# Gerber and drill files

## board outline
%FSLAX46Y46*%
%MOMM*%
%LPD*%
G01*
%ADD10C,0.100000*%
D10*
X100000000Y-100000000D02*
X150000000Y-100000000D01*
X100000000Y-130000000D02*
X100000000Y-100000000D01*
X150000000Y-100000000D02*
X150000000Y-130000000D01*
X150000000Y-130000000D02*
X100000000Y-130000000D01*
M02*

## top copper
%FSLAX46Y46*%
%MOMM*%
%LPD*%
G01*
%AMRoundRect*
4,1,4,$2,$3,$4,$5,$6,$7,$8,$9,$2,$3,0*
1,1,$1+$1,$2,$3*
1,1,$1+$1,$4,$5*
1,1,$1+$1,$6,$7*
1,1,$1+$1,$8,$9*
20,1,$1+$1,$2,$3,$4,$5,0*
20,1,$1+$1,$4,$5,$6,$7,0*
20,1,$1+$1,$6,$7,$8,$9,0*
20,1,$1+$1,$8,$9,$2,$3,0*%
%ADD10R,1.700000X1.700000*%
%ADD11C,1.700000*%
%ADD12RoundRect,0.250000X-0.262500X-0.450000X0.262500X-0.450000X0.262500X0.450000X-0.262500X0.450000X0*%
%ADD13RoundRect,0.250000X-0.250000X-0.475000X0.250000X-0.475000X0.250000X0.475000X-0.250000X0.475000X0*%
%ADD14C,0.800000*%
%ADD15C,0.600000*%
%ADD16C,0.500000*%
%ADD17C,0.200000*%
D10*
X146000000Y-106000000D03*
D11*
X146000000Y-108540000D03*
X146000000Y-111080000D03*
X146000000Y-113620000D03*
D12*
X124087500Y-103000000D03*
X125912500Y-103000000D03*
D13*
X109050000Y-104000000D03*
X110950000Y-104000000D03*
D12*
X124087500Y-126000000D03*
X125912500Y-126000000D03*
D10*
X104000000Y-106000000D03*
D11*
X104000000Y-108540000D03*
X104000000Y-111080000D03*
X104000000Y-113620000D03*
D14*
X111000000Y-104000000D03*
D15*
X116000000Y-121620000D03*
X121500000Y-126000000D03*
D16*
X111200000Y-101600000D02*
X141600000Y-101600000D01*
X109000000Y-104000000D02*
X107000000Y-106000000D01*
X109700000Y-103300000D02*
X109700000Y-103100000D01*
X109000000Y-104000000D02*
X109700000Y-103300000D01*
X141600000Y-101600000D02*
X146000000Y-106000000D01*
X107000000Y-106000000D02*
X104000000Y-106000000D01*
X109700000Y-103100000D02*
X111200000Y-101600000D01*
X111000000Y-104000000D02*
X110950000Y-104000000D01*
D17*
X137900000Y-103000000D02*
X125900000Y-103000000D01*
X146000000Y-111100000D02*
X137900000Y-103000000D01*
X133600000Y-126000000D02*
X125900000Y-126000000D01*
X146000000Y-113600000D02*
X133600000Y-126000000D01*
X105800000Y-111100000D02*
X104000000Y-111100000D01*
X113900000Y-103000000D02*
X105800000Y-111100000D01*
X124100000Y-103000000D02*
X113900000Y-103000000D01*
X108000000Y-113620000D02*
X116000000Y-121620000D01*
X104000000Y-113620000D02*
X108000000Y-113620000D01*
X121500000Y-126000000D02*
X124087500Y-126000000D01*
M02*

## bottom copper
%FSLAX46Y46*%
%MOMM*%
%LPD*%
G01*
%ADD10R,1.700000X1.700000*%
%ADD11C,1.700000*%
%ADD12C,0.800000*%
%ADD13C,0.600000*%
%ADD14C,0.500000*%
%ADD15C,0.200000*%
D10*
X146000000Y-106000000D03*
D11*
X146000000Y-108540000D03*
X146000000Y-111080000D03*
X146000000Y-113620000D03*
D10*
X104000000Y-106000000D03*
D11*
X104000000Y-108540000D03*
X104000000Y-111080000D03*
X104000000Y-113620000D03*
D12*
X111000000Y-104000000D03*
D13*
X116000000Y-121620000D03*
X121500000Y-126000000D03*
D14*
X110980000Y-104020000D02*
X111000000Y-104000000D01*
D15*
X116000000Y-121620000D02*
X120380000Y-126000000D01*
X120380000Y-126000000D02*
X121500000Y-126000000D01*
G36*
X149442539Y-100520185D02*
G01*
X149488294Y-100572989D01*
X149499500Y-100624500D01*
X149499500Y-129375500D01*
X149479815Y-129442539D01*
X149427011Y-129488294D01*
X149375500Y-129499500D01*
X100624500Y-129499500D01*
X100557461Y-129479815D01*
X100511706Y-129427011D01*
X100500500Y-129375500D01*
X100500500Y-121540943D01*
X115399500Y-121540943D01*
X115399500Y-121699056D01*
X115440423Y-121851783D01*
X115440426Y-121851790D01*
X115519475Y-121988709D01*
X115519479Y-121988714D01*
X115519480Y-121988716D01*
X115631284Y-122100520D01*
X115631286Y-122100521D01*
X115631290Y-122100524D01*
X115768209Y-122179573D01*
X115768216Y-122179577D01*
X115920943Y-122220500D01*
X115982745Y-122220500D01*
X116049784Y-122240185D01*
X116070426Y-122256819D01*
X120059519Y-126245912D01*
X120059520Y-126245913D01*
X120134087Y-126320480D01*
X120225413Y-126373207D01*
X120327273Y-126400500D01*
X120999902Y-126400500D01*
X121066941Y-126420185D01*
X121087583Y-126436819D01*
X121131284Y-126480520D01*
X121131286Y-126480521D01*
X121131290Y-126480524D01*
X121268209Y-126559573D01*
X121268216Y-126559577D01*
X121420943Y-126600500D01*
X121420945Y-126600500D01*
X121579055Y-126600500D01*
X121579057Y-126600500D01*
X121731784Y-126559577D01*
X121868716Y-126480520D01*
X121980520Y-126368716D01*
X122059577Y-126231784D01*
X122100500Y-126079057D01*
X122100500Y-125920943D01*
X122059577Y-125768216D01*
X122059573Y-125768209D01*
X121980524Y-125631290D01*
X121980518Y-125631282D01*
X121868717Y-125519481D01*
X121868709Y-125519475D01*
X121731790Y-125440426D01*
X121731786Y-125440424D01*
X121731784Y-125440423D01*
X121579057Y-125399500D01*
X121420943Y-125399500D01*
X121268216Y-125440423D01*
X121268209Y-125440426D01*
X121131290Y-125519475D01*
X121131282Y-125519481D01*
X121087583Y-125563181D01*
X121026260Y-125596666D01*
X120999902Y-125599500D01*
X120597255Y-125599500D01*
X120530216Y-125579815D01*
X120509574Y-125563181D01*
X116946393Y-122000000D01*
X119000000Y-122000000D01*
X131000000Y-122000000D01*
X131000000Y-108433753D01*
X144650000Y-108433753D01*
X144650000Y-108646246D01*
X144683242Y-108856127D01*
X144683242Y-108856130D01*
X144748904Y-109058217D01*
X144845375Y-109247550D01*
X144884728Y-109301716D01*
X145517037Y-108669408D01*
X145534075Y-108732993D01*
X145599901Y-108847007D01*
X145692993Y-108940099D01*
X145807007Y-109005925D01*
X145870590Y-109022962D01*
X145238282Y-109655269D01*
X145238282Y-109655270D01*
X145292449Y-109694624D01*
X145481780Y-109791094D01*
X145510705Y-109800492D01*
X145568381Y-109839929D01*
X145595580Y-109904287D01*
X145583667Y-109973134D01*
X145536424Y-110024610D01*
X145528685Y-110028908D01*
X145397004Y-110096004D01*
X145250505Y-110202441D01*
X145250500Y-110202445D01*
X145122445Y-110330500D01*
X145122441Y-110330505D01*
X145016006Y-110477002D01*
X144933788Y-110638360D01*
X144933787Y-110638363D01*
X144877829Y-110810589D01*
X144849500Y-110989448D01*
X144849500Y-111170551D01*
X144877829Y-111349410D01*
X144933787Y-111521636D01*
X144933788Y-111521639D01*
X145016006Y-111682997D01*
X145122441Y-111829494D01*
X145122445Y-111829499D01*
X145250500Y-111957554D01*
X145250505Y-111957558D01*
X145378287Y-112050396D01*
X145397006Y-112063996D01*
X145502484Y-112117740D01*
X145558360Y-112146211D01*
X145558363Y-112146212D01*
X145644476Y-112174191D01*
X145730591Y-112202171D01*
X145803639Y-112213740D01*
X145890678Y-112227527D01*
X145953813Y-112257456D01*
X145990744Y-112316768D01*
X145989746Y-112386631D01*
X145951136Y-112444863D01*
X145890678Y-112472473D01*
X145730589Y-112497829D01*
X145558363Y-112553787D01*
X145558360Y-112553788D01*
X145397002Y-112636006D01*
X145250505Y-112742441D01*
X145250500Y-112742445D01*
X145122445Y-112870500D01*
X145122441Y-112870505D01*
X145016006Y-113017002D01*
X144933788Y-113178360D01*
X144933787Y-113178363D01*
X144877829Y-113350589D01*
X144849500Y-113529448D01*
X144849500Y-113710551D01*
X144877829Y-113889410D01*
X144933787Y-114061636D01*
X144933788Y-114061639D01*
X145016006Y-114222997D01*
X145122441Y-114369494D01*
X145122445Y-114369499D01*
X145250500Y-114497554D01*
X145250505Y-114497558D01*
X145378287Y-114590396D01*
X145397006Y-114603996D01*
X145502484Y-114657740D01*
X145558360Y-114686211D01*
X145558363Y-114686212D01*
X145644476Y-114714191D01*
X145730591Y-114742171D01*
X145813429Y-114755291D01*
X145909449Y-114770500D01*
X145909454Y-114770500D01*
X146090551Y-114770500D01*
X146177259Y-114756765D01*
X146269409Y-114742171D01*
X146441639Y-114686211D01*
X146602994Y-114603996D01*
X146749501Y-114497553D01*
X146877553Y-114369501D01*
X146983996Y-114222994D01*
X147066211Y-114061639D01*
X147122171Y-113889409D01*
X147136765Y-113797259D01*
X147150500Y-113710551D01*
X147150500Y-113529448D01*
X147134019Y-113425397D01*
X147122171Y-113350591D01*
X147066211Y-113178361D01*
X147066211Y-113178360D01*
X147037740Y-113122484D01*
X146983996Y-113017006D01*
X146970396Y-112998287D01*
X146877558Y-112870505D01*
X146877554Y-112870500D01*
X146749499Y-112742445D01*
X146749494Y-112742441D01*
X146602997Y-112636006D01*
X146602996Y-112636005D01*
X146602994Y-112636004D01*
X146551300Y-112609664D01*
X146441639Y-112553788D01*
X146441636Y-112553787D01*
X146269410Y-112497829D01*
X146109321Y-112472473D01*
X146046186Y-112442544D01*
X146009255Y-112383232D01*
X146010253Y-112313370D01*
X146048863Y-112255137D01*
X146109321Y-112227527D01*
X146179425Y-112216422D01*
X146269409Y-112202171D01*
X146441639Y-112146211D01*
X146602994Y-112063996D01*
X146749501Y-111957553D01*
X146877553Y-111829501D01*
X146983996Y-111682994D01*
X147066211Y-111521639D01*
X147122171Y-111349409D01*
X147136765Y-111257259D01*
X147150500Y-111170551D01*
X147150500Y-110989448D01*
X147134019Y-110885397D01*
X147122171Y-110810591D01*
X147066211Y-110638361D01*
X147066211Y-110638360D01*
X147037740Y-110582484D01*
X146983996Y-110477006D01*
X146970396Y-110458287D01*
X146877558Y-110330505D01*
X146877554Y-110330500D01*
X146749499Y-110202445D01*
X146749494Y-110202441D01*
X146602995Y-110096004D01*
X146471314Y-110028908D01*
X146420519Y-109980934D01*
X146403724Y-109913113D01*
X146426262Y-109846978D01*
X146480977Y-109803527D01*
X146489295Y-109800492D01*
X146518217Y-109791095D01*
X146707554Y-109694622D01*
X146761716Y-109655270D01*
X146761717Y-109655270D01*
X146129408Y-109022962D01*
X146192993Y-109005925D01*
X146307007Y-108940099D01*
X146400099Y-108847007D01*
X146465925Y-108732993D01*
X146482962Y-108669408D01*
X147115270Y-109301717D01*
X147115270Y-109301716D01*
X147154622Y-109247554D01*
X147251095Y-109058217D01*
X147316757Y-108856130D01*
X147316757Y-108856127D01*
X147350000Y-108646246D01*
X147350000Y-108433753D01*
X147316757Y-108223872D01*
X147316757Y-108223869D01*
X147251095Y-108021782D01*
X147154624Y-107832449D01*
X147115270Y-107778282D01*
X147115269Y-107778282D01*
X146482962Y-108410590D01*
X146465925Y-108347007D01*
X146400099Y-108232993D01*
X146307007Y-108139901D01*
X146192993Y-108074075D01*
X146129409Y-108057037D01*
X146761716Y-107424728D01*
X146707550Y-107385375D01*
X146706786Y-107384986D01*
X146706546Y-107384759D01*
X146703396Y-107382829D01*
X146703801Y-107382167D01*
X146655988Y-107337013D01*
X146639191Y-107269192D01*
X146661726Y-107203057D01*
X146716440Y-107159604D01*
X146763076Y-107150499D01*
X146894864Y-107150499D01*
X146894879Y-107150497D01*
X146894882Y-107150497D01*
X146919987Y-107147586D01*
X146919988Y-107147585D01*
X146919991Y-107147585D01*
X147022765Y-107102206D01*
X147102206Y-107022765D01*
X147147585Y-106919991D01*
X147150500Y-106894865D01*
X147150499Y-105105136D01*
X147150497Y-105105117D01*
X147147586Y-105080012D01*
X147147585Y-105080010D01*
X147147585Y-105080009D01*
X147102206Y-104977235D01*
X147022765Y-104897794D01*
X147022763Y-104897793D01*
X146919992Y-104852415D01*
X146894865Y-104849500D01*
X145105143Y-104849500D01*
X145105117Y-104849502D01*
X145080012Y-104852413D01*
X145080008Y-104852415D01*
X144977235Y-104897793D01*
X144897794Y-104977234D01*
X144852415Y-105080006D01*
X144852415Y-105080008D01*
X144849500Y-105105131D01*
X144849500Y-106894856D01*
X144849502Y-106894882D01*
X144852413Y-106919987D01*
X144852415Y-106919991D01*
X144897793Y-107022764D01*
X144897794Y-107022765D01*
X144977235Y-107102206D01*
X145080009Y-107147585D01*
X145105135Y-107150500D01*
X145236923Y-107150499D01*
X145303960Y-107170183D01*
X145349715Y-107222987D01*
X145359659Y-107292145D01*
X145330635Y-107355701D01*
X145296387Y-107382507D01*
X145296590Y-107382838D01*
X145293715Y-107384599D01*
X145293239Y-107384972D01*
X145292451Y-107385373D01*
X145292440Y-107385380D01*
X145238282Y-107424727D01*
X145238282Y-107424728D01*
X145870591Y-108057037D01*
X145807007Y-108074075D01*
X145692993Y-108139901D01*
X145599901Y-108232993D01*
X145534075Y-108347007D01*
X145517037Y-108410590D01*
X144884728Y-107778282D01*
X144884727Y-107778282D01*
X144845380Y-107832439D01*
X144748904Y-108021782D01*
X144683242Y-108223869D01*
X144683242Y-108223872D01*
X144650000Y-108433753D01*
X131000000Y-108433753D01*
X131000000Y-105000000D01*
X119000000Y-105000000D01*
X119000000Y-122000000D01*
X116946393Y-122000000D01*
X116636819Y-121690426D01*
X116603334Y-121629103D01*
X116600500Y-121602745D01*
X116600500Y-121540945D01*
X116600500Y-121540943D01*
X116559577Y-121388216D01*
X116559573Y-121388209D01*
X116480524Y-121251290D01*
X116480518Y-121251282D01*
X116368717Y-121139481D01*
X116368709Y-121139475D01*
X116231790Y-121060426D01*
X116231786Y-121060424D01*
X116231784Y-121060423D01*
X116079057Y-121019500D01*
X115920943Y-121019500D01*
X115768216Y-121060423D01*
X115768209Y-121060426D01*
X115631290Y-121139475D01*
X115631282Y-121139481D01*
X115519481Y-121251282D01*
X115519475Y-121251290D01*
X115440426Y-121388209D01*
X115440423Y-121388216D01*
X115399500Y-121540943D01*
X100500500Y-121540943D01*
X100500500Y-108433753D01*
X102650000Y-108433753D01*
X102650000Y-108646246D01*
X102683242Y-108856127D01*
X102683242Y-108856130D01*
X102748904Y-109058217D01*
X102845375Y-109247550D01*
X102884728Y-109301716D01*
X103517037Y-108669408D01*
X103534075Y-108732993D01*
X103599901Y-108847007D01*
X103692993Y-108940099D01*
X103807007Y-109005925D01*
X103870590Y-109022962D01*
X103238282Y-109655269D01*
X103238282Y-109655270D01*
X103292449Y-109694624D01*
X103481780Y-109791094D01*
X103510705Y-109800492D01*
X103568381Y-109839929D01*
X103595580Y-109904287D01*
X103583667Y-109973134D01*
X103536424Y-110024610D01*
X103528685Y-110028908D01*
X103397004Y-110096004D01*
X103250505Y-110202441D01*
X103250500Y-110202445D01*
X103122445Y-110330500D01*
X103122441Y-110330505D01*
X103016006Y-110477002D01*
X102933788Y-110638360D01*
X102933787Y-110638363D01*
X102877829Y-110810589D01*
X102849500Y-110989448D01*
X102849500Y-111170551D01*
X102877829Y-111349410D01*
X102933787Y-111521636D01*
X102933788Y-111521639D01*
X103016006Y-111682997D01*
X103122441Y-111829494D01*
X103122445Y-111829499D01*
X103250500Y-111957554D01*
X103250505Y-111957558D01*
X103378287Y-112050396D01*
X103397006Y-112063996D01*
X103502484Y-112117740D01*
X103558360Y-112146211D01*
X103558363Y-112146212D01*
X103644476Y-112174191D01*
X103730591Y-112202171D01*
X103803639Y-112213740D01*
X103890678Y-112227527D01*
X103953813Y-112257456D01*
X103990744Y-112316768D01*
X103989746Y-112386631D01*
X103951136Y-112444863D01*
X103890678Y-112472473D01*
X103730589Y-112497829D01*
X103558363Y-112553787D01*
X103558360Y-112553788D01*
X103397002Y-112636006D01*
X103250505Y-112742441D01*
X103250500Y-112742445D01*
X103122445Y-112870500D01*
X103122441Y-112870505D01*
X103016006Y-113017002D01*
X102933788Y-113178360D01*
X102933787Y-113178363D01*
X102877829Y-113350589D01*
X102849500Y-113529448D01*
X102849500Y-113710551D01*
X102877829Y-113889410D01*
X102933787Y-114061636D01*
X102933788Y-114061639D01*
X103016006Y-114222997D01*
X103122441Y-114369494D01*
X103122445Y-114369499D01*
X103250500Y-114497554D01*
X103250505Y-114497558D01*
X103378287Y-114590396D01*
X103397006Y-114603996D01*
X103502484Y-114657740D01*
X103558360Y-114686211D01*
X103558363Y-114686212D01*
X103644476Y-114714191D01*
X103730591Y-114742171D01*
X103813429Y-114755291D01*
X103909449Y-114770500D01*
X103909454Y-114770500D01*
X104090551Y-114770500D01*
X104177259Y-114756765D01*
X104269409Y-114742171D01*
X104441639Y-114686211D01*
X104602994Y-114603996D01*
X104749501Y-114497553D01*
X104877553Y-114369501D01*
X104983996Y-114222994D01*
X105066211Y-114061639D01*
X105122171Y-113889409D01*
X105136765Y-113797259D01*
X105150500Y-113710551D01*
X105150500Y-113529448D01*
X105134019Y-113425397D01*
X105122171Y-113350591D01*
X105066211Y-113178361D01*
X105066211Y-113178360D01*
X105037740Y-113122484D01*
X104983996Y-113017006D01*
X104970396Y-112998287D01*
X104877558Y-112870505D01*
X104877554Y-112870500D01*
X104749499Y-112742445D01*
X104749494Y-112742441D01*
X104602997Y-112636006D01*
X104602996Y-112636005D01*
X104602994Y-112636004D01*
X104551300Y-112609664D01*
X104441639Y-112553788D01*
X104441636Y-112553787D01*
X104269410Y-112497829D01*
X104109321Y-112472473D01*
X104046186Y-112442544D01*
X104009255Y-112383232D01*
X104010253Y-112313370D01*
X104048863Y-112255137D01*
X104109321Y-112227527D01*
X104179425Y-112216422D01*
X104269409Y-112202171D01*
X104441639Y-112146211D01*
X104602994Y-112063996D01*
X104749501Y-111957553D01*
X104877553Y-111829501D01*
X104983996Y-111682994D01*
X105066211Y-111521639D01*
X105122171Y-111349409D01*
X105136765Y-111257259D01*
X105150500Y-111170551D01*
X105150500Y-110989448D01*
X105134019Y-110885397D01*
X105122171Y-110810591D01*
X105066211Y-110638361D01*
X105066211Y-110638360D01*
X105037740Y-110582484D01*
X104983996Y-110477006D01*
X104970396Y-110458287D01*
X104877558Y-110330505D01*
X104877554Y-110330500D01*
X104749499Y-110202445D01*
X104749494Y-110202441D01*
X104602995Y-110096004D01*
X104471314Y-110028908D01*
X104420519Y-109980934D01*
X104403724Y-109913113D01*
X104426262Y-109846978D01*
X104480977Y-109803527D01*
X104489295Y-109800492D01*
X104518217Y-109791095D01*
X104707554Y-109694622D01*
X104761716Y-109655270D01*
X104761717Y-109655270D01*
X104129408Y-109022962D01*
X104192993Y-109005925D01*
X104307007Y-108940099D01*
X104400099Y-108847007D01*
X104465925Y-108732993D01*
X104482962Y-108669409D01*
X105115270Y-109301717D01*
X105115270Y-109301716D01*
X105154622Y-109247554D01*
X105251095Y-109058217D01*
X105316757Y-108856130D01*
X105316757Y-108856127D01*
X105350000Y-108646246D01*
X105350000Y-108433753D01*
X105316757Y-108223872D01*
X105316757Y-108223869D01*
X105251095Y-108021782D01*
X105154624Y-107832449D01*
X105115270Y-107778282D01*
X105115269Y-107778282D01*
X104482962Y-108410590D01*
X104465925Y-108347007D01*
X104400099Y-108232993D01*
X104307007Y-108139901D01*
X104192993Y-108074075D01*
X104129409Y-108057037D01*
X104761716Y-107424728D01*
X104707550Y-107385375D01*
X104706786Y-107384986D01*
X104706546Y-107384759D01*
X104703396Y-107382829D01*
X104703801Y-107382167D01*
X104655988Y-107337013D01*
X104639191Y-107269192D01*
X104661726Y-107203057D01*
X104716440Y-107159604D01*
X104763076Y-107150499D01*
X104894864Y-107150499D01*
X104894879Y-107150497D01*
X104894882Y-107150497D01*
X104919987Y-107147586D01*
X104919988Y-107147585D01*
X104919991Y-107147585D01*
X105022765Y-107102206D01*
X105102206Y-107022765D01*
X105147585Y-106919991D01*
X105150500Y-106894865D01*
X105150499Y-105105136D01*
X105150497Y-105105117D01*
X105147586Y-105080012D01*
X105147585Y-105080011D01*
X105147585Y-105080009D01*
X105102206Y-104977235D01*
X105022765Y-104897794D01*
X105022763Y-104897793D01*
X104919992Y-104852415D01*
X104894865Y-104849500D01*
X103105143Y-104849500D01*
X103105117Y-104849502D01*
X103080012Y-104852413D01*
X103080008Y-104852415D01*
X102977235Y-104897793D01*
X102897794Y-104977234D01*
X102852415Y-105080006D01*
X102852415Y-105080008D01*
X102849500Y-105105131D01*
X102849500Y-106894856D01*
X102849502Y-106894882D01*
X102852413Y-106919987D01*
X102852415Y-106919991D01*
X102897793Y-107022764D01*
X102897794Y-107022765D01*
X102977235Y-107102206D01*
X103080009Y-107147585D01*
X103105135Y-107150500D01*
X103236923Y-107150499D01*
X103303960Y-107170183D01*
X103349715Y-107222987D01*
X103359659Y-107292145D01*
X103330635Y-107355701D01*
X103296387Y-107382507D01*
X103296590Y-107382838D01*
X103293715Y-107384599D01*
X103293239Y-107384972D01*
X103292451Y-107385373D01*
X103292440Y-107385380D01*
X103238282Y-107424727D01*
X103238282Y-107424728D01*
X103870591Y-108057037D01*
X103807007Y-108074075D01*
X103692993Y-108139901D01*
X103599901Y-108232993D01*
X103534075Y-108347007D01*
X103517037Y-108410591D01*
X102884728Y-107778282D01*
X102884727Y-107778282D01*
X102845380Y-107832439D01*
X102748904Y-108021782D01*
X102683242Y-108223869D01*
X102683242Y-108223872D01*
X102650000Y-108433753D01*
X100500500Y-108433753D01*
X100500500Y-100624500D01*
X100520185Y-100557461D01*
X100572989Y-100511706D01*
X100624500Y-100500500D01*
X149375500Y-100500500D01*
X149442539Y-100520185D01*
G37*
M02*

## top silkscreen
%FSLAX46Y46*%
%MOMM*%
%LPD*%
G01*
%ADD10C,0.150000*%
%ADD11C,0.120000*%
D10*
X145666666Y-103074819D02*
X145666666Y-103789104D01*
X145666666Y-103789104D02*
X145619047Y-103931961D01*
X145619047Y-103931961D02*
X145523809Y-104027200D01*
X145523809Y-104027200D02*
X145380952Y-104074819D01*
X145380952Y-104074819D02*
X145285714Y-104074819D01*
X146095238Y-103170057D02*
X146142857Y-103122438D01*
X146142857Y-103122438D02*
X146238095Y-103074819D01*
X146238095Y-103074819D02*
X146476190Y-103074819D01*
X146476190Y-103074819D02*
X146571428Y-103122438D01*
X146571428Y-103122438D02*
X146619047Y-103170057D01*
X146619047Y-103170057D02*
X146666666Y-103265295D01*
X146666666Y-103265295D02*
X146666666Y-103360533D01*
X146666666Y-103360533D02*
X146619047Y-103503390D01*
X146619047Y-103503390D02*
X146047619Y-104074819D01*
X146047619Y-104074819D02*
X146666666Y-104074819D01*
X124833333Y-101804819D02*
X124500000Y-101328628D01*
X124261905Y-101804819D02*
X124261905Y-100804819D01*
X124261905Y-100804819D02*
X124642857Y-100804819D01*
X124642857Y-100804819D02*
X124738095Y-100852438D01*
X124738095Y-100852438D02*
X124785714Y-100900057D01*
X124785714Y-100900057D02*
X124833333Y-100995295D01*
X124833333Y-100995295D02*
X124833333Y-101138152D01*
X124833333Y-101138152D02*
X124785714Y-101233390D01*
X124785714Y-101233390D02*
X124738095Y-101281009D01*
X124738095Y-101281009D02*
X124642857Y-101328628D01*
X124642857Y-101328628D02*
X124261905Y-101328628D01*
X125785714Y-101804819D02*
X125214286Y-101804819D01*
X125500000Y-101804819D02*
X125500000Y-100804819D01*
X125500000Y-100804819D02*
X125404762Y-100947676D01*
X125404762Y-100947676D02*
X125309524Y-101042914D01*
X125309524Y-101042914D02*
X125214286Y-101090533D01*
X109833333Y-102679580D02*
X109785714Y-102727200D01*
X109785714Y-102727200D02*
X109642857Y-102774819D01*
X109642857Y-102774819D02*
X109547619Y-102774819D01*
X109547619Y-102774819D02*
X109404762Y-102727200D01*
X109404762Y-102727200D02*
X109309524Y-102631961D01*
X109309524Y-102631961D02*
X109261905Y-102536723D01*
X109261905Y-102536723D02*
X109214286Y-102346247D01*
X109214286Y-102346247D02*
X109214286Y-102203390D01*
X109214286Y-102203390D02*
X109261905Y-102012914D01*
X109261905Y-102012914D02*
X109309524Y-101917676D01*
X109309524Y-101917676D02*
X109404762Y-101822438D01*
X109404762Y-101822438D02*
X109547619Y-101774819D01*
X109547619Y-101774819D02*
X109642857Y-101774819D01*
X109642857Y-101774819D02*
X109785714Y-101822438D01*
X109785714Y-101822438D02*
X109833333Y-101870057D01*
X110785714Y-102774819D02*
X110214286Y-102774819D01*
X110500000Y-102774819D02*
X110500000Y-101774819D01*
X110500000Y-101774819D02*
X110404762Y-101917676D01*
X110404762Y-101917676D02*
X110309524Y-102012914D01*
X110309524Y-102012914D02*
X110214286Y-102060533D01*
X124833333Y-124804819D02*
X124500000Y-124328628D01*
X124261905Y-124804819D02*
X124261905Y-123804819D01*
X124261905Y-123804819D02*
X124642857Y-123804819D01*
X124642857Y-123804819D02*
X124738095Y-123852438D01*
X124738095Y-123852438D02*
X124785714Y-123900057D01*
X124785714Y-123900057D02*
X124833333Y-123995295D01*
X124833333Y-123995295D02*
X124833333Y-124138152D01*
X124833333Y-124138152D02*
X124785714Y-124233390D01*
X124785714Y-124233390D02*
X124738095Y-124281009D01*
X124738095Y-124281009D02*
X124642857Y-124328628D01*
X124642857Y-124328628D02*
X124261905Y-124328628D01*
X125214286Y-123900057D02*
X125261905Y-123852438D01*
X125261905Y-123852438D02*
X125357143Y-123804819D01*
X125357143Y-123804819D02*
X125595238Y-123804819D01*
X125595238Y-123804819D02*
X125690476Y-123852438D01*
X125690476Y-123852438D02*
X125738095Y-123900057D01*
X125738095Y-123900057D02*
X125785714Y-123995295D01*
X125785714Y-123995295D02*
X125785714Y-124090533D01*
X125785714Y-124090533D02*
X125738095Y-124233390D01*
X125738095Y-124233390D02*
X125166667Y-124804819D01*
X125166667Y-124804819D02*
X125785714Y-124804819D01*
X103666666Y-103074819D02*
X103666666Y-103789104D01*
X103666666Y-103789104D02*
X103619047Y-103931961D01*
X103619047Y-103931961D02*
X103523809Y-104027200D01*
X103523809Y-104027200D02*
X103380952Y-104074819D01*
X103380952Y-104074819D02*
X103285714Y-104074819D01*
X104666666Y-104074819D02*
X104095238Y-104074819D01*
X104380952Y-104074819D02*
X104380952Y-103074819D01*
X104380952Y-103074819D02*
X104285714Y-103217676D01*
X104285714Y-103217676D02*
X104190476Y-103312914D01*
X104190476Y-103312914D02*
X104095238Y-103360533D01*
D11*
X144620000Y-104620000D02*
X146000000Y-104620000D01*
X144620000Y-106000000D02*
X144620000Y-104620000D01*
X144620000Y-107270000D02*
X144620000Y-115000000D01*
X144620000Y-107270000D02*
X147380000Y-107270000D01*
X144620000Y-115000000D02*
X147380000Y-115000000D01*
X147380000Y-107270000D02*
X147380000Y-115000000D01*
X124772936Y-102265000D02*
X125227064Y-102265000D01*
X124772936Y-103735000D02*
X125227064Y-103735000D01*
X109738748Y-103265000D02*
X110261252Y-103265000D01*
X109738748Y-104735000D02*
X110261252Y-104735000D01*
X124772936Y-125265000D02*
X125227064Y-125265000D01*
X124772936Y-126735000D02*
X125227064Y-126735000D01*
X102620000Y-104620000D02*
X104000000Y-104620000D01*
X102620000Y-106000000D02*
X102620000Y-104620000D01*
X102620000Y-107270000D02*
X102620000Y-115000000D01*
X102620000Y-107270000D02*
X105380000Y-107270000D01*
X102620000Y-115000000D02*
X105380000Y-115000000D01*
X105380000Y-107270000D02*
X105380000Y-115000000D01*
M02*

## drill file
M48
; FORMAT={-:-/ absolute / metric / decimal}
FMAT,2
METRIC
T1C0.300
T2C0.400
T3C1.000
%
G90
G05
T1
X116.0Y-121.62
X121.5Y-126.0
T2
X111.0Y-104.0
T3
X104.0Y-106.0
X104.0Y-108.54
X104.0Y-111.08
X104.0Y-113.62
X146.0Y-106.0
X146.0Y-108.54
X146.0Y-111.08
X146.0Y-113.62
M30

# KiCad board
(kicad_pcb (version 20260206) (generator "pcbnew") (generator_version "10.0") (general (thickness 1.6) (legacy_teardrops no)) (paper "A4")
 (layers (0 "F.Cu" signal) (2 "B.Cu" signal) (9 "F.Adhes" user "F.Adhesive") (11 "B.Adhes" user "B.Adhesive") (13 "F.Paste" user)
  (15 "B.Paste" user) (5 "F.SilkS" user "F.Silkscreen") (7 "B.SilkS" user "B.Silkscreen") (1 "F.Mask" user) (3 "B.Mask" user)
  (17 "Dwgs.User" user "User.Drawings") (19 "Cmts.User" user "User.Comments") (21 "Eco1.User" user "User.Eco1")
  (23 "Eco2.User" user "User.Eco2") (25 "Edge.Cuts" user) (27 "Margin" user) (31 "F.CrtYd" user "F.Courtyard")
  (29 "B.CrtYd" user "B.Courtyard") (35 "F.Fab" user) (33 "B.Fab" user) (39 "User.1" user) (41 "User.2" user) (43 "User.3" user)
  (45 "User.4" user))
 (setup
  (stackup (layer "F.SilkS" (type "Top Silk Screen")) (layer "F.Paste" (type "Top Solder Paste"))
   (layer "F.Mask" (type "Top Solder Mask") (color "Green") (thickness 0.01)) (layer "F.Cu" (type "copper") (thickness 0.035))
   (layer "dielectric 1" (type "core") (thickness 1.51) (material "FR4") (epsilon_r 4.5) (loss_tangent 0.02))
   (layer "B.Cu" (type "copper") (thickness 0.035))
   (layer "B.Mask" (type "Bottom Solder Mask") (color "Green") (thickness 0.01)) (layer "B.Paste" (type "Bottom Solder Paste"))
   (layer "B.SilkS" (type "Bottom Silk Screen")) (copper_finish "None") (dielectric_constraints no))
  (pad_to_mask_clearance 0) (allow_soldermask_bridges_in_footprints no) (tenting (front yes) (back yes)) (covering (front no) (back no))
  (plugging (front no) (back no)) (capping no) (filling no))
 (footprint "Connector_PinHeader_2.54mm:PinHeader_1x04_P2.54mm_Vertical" (layer "F.Cu") (at 146 106)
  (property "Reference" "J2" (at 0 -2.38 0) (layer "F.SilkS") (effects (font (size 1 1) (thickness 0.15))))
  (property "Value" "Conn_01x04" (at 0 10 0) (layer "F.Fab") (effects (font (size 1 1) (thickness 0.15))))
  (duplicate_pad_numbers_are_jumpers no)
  (fp_line (start -1.38 -1.38) (end 0 -1.38) (stroke (width 0.12) (type solid)) (layer "F.SilkS"))
  (fp_line (start -1.38 0) (end -1.38 -1.38) (stroke (width 0.12) (type solid)) (layer "F.SilkS"))
  (fp_line (start -1.38 1.27) (end -1.38 9) (stroke (width 0.12) (type solid)) (layer "F.SilkS"))
  (fp_line (start -1.38 1.27) (end 1.38 1.27) (stroke (width 0.12) (type solid)) (layer "F.SilkS"))
  (fp_line (start -1.38 9) (end 1.38 9) (stroke (width 0.12) (type solid)) (layer "F.SilkS"))
  (fp_line (start 1.38 1.27) (end 1.38 9) (stroke (width 0.12) (type solid)) (layer "F.SilkS"))
  (pad "1" thru_hole rect (at 0 0) (size 1.7 1.7) (drill 1) (layers "*.Cu" "*.Mask") (remove_unused_layers no) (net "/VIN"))
  (pad "2" thru_hole circle (at 0 2.54) (size 1.7 1.7) (drill 1) (layers "*.Cu" "*.Mask") (remove_unused_layers no) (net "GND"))
  (pad "3" thru_hole circle (at 0 5.08) (size 1.7 1.7) (drill 1) (layers "*.Cu" "*.Mask") (remove_unused_layers no) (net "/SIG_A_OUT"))
  (pad "4" thru_hole circle (at 0 7.62) (size 1.7 1.7) (drill 1) (layers "*.Cu" "*.Mask") (remove_unused_layers no) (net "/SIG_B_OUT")))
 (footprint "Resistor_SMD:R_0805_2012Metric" (layer "F.Cu") (at 125 103)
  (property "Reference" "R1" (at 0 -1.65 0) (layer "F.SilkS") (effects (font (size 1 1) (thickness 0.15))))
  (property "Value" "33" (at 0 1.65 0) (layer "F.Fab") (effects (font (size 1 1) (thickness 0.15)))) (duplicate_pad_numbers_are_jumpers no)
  (fp_line (start -0.227064 -0.735) (end 0.227064 -0.735) (stroke (width 0.12) (type solid)) (layer "F.SilkS"))
  (fp_line (start -0.227064 0.735) (end 0.227064 0.735) (stroke (width 0.12) (type solid)) (layer "F.SilkS"))
  (pad "1" smd roundrect (at -0.9125 0) (size 1.025 1.4) (layers "F.Cu" "F.Mask" "F.Paste") (roundrect_rratio 0.243902) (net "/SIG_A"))
  (pad "2" smd roundrect (at 0.9125 0) (size 1.025 1.4) (layers "F.Cu" "F.Mask" "F.Paste") (roundrect_rratio 0.243902) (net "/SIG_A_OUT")))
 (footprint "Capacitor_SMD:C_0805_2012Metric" (layer "F.Cu") (at 110 104)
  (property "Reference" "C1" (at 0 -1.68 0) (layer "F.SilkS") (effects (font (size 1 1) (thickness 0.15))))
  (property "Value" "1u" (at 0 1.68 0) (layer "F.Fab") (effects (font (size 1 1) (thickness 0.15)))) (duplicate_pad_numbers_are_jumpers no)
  (fp_line (start -0.261252 -0.735) (end 0.261252 -0.735) (stroke (width 0.12) (type solid)) (layer "F.SilkS"))
  (fp_line (start -0.261252 0.735) (end 0.261252 0.735) (stroke (width 0.12) (type solid)) (layer "F.SilkS"))
  (pad "1" smd roundrect (at -0.95 0) (size 1 1.45) (layers "F.Cu" "F.Mask" "F.Paste") (roundrect_rratio 0.25) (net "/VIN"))
  (pad "2" smd roundrect (at 0.95 0) (size 1 1.45) (layers "F.Cu" "F.Mask" "F.Paste") (roundrect_rratio 0.25) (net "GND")))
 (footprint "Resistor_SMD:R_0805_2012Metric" (layer "F.Cu") (at 125 126)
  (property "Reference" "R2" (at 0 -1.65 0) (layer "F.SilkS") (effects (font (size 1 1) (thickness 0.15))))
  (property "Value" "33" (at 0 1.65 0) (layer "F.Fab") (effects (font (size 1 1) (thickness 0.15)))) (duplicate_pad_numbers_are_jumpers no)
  (fp_line (start -0.227064 -0.735) (end 0.227064 -0.735) (stroke (width 0.12) (type solid)) (layer "F.SilkS"))
  (fp_line (start -0.227064 0.735) (end 0.227064 0.735) (stroke (width 0.12) (type solid)) (layer "F.SilkS"))
  (pad "1" smd roundrect (at -0.9125 0) (size 1.025 1.4) (layers "F.Cu" "F.Mask" "F.Paste") (roundrect_rratio 0.243902) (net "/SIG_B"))
  (pad "2" smd roundrect (at 0.9125 0) (size 1.025 1.4) (layers "F.Cu" "F.Mask" "F.Paste") (roundrect_rratio 0.243902) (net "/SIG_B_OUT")))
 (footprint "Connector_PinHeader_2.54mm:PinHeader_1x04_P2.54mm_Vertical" (layer "F.Cu") (at 104 106)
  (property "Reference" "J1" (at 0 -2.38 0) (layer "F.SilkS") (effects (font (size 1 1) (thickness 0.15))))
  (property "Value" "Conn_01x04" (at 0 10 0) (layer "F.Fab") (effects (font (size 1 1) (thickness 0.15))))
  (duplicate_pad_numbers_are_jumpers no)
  (fp_line (start -1.38 -1.38) (end 0 -1.38) (stroke (width 0.12) (type solid)) (layer "F.SilkS"))
  (fp_line (start -1.38 0) (end -1.38 -1.38) (stroke (width 0.12) (type solid)) (layer "F.SilkS"))
  (fp_line (start -1.38 1.27) (end -1.38 9) (stroke (width 0.12) (type solid)) (layer "F.SilkS"))
  (fp_line (start -1.38 1.27) (end 1.38 1.27) (stroke (width 0.12) (type solid)) (layer "F.SilkS"))
  (fp_line (start -1.38 9) (end 1.38 9) (stroke (width 0.12) (type solid)) (layer "F.SilkS"))
  (fp_line (start 1.38 1.27) (end 1.38 9) (stroke (width 0.12) (type solid)) (layer "F.SilkS"))
  (pad "1" thru_hole rect (at 0 0) (size 1.7 1.7) (drill 1) (layers "*.Cu" "*.Mask") (remove_unused_layers no) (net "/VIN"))
  (pad "2" thru_hole circle (at 0 2.54) (size 1.7 1.7) (drill 1) (layers "*.Cu" "*.Mask") (remove_unused_layers no) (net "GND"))
  (pad "3" thru_hole circle (at 0 5.08) (size 1.7 1.7) (drill 1) (layers "*.Cu" "*.Mask") (remove_unused_layers no) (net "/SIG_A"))
  (pad "4" thru_hole circle (at 0 7.62) (size 1.7 1.7) (drill 1) (layers "*.Cu" "*.Mask") (remove_unused_layers no) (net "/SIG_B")))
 (gr_line (start 100 100) (end 150 100) (stroke (width 0.1) (type default)) (layer "Edge.Cuts"))
 (gr_line (start 100 130) (end 100 100) (stroke (width 0.1) (type default)) (layer "Edge.Cuts"))
 (gr_line (start 150 100) (end 150 130) (stroke (width 0.1) (type default)) (layer "Edge.Cuts"))
 (gr_line (start 150 130) (end 100 130) (stroke (width 0.1) (type default)) (layer "Edge.Cuts"))
 (segment (start 111.2 101.6) (end 141.6 101.6) (width 0.5) (layer "F.Cu") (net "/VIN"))
 (segment (start 109 104) (end 107 106) (width 0.5) (layer "F.Cu") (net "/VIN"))
 (segment (start 109.7 103.3) (end 109.7 103.1) (width 0.5) (layer "F.Cu") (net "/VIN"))
 (segment (start 109 104) (end 109.7 103.3) (width 0.5) (layer "F.Cu") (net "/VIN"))
 (segment (start 141.6 101.6) (end 146 106) (width 0.5) (layer "F.Cu") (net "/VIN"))
 (segment (start 107 106) (end 104 106) (width 0.5) (layer "F.Cu") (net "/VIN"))
 (segment (start 109.7 103.1) (end 111.2 101.6) (width 0.5) (layer "F.Cu") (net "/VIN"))
 (segment (start 111 104) (end 110.95 104) (width 0.5) (layer "F.Cu") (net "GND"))
 (via (at 111 104) (size 0.8) (drill 0.4) (layers "F.Cu" "B.Cu") (capping yes) (filling yes) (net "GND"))
 (segment (start 110.98 104.02) (end 111 104) (width 0.5) (layer "B.Cu") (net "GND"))
 (segment (start 137.9 103) (end 125.9 103) (width 0.2) (layer "F.Cu") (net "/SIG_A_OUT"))
 (segment (start 146 111.1) (end 137.9 103) (width 0.2) (layer "F.Cu") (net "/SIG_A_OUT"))
 (segment (start 133.6 126) (end 125.9 126) (width 0.2) (layer "F.Cu") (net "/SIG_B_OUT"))
 (segment (start 146 113.6) (end 133.6 126) (width 0.2) (layer "F.Cu") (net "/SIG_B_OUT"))
 (segment (start 105.8 111.1) (end 104 111.1) (width 0.2) (layer "F.Cu") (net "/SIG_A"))
 (segment (start 113.9 103) (end 105.8 111.1) (width 0.2) (layer "F.Cu") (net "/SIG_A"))
 (segment (start 124.1 103) (end 113.9 103) (width 0.2) (layer "F.Cu") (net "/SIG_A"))
 (segment (start 108 113.62) (end 116 121.62) (width 0.2) (locked yes) (layer "F.Cu") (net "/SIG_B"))
 (segment (start 104 113.62) (end 108 113.62) (width 0.2) (locked yes) (layer "F.Cu") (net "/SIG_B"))
 (segment (start 121.5 126) (end 124.0875 126) (width 0.2) (locked yes) (layer "F.Cu") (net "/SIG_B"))
 (via (at 116 121.62) (size 0.6) (drill 0.3) (layers "F.Cu" "B.Cu") (locked yes) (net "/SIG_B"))
 (via (at 121.5 126) (size 0.6) (drill 0.3) (layers "F.Cu" "B.Cu") (locked yes) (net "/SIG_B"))
 (segment (start 116 121.62) (end 120.38 126) (width 0.2) (locked yes) (layer "B.Cu") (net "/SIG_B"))
 (segment (start 120.38 126) (end 121.5 126) (width 0.2) (locked yes) (layer "B.Cu") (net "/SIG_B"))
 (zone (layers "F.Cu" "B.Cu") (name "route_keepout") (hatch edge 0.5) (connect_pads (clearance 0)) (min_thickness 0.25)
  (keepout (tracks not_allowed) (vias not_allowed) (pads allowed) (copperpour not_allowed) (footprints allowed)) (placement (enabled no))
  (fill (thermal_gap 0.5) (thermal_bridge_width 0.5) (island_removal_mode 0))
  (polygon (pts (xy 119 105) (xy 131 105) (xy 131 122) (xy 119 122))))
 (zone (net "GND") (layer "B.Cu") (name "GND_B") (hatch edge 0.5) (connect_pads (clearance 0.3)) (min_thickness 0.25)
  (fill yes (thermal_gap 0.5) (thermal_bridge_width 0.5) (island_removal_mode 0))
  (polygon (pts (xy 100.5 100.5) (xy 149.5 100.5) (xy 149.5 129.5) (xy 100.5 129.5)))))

